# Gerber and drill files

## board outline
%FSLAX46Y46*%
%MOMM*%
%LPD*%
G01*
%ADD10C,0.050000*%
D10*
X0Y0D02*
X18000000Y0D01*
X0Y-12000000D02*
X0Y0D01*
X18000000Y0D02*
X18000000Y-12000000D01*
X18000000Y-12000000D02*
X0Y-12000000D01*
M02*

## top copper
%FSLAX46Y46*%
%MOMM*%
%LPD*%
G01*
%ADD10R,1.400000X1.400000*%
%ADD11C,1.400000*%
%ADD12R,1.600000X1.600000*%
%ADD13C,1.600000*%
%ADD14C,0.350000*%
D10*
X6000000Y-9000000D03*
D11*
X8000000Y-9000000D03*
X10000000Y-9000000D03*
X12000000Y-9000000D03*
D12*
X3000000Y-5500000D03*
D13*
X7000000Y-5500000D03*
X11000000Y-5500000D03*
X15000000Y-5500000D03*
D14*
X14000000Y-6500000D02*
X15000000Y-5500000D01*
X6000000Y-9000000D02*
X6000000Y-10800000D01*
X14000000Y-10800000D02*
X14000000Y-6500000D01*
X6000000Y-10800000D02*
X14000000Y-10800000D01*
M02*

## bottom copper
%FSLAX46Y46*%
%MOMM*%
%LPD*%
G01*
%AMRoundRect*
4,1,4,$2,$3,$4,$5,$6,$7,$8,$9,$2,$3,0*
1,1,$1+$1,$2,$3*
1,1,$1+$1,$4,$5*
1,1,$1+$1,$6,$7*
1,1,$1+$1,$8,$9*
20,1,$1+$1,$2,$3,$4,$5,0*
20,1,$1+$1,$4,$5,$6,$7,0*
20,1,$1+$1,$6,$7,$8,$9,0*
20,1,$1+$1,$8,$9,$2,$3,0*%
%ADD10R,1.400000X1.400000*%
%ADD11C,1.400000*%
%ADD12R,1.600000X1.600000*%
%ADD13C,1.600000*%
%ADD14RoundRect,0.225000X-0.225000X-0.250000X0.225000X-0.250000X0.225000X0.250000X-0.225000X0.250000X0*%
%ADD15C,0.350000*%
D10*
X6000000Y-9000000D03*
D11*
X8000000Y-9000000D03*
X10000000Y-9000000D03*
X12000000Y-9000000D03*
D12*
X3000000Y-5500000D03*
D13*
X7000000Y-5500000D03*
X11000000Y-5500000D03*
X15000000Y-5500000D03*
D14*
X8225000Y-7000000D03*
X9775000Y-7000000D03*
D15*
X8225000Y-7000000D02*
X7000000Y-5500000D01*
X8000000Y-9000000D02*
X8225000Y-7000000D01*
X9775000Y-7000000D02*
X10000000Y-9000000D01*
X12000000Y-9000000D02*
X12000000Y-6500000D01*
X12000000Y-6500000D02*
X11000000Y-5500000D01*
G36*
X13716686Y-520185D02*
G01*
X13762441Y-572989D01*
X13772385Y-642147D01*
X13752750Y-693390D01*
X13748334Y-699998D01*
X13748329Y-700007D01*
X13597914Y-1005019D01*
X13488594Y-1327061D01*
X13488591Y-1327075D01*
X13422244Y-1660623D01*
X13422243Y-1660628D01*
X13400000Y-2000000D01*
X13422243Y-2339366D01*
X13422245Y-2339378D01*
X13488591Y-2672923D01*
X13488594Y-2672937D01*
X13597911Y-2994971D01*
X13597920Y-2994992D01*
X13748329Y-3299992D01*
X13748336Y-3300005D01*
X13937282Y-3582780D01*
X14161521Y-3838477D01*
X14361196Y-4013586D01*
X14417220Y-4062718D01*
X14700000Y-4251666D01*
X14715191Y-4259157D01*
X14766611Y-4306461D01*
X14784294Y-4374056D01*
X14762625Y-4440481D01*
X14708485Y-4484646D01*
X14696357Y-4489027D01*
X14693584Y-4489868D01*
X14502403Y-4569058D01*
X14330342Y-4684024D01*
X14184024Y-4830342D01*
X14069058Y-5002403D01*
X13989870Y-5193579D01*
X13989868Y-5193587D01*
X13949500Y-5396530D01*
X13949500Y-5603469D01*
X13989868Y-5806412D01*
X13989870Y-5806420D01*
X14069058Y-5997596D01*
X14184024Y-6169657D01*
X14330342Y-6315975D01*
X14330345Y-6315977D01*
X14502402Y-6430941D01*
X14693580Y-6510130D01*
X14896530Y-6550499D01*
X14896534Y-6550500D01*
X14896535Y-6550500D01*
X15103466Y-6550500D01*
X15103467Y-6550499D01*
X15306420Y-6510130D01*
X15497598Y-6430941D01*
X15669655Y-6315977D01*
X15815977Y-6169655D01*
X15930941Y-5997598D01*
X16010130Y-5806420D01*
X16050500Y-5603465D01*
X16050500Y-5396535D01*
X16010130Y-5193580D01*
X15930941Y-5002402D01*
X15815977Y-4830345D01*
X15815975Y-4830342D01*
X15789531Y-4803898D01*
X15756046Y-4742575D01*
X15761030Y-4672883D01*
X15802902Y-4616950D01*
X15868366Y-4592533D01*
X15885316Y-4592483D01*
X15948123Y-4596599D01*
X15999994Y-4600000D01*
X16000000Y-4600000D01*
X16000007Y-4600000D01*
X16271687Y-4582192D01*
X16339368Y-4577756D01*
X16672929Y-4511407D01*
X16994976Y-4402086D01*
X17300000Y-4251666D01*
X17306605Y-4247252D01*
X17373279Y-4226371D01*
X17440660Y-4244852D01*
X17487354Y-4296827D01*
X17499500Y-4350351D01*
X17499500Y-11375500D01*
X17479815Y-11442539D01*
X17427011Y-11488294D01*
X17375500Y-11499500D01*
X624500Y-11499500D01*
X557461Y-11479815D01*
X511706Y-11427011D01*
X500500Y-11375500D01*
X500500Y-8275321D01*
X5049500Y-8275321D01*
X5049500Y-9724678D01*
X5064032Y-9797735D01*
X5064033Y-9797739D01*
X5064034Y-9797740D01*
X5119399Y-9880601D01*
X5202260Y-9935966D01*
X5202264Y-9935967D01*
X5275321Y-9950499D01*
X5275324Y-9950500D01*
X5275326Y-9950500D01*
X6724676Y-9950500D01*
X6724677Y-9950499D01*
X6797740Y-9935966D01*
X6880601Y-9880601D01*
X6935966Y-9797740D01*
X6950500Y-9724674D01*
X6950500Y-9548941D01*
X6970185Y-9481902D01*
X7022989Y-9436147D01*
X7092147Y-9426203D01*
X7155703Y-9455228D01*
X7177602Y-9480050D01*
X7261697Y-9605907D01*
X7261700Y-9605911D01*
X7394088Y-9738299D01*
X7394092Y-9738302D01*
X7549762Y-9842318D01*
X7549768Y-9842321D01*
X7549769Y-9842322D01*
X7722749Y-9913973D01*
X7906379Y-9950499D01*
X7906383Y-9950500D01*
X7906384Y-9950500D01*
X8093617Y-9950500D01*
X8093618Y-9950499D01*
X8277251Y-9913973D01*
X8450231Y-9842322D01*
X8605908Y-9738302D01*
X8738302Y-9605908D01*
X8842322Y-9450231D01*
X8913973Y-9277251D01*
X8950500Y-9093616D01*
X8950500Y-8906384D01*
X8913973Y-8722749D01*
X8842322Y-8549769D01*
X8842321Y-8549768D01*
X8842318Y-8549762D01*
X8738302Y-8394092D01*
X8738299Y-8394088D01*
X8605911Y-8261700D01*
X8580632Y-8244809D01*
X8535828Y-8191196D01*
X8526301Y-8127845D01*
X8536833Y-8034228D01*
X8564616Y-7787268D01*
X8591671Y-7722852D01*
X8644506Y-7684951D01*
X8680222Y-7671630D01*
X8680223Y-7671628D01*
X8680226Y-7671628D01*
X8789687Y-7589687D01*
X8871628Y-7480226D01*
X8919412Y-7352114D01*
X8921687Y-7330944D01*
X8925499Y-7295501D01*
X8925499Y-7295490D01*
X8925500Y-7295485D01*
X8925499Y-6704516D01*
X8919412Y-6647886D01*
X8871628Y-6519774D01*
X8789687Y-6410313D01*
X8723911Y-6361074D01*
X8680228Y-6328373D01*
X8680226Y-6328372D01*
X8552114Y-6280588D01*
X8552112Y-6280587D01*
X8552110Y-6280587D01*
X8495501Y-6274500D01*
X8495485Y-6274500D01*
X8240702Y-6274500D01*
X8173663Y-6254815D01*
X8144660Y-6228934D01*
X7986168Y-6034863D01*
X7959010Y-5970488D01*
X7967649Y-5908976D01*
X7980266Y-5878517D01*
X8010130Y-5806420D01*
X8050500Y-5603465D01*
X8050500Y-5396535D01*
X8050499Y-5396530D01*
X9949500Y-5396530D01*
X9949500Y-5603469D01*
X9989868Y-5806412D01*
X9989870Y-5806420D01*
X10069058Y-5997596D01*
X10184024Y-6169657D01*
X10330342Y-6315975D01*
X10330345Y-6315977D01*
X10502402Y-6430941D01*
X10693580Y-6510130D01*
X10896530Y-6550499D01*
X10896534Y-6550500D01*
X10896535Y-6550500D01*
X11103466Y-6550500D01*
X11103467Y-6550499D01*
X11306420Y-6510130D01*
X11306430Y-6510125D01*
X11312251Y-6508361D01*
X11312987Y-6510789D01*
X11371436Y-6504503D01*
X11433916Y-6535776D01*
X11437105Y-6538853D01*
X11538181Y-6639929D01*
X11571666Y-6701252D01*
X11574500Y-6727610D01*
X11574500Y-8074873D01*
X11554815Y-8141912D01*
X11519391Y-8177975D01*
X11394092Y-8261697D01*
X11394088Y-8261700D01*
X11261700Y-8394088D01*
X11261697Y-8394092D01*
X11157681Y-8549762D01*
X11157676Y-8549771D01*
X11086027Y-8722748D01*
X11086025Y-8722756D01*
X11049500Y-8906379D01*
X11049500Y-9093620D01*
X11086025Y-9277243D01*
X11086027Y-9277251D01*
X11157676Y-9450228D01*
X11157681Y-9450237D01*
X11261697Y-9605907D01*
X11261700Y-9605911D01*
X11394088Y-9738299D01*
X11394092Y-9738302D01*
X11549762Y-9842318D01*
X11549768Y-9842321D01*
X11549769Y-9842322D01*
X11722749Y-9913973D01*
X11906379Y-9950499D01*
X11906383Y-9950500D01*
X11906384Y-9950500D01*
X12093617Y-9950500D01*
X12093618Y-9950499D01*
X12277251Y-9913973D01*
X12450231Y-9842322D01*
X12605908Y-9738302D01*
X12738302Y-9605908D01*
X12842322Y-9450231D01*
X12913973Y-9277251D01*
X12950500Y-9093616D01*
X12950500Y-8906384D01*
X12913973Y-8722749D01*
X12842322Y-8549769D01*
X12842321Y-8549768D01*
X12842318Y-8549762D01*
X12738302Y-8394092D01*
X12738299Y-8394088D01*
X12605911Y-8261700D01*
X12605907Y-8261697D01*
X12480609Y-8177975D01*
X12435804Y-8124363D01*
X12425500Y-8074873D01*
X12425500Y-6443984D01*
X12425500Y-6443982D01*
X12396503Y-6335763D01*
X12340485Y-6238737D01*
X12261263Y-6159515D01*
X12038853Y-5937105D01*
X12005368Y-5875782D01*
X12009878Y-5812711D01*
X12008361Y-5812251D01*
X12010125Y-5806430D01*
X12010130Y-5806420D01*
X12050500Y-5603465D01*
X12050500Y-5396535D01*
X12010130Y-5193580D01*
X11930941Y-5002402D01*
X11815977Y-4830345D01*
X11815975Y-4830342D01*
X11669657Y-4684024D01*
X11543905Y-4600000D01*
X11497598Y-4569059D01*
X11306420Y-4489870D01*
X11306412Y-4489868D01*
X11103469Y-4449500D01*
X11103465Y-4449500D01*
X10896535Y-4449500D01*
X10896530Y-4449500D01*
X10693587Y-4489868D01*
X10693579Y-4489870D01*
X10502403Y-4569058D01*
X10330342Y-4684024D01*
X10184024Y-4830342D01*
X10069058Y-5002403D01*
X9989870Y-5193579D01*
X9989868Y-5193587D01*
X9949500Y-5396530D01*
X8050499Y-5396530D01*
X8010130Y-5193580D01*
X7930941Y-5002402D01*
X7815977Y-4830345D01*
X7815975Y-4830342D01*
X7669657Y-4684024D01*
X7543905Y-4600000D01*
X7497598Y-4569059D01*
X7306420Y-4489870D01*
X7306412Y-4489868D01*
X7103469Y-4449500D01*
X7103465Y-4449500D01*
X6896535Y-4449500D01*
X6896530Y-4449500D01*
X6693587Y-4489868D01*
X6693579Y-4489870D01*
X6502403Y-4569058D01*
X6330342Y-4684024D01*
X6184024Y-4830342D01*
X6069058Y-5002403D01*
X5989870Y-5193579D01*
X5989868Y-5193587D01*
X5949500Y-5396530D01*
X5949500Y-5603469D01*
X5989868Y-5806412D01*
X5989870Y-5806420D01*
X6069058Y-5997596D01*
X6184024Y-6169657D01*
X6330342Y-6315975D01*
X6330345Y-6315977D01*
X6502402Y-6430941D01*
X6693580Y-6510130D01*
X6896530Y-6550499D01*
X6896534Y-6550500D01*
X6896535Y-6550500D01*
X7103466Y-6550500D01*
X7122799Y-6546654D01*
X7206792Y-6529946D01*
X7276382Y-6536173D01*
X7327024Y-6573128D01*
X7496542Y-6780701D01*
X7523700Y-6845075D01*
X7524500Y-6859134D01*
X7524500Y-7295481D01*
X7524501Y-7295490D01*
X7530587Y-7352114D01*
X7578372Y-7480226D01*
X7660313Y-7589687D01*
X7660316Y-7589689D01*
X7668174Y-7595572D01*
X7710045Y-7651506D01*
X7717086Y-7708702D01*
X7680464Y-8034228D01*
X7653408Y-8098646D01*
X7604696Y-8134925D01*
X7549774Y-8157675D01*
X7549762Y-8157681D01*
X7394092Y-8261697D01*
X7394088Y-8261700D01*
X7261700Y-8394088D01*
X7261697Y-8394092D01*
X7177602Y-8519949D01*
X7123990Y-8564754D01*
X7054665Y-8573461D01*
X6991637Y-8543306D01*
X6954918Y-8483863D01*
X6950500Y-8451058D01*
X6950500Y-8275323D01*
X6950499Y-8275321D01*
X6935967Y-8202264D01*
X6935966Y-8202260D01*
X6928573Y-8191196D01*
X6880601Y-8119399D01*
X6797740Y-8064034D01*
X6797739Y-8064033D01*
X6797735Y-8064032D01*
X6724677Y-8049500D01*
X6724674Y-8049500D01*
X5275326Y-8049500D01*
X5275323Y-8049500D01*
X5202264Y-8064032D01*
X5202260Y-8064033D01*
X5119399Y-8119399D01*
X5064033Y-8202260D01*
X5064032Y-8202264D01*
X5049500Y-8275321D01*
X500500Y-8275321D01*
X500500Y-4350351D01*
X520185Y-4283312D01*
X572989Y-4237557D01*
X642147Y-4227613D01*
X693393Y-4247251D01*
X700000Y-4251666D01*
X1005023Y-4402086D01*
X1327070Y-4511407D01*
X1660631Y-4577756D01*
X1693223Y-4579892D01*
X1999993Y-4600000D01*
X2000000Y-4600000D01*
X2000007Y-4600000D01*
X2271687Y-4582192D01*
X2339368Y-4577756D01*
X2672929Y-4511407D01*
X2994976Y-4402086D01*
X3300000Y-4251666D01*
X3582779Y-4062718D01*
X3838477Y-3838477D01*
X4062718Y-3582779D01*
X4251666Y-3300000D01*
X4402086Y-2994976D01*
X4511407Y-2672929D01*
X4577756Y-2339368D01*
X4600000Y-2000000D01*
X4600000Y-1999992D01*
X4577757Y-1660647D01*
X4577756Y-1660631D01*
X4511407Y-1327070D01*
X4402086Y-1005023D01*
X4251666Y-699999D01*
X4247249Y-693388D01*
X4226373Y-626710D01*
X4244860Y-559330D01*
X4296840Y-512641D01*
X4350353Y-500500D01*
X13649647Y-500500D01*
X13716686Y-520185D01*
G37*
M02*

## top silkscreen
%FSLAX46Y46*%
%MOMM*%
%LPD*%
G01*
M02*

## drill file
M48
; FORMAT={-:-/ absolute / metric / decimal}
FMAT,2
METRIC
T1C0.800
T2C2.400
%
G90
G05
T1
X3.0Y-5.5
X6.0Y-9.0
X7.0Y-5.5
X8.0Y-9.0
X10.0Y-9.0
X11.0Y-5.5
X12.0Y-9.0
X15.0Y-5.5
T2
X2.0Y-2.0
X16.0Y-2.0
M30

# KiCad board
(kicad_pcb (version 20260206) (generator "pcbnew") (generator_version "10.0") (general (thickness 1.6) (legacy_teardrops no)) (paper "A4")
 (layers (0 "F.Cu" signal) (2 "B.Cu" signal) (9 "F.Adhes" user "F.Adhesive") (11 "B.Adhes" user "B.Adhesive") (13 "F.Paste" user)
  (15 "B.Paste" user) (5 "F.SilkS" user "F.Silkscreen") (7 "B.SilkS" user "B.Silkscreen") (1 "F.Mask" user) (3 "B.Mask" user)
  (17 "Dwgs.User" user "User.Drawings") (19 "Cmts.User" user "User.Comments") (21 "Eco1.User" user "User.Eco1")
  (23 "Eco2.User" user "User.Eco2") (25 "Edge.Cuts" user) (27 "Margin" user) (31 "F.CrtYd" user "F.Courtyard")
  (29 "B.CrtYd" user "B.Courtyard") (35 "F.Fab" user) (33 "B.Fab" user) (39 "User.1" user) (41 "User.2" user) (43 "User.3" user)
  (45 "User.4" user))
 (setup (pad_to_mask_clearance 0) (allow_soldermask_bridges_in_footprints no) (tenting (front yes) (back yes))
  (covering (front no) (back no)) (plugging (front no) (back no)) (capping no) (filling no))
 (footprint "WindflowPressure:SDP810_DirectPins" (layer "F.Cu") (at 9 6)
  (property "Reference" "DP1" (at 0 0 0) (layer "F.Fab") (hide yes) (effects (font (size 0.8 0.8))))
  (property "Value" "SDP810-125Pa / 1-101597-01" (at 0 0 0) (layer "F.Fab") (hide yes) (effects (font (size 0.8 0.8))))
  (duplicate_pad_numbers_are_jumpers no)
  (pad "1" thru_hole rect (at -3 3) (size 1.4 1.4) (drill 0.8) (layers "*.Cu" "*.Mask") (remove_unused_layers no) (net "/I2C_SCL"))
  (pad "2" thru_hole circle (at -1 3) (size 1.4 1.4) (drill 0.8) (layers "*.Cu" "*.Mask") (remove_unused_layers no) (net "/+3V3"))
  (pad "3" thru_hole circle (at 1 3) (size 1.4 1.4) (drill 0.8) (layers "*.Cu" "*.Mask") (remove_unused_layers no) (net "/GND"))
  (pad "4" thru_hole circle (at 3 3) (size 1.4 1.4) (drill 0.8) (layers "*.Cu" "*.Mask") (remove_unused_layers no) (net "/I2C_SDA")))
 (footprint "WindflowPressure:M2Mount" (layer "F.Cu") (at 2 2)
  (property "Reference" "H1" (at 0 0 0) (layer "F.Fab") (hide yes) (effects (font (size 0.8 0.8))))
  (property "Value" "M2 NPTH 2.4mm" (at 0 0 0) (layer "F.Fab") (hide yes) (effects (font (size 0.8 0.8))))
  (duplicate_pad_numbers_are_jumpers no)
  (pad "" np_thru_hole circle (at 0 0) (size 2.4 2.4) (drill 2.4) (layers "*.Cu" "*.Mask")))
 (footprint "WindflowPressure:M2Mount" (layer "F.Cu") (at 16 2)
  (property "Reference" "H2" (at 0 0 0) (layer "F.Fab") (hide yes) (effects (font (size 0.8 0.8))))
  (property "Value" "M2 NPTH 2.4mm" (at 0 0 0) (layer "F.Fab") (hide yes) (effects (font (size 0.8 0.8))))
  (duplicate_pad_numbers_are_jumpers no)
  (pad "" np_thru_hole circle (at 0 0) (size 2.4 2.4) (drill 2.4) (layers "*.Cu" "*.Mask")))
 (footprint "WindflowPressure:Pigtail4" (layer "F.Cu") (at 9 5.5)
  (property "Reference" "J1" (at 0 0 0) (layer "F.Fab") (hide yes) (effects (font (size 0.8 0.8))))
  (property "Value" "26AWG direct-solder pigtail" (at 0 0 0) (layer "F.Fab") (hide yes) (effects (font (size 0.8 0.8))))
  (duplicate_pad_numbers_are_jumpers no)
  (pad "1" thru_hole rect (at -6 0) (size 1.6 1.6) (drill 0.8) (layers "*.Cu" "*.Mask") (remove_unused_layers no) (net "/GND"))
  (pad "2" thru_hole circle (at -2 0) (size 1.6 1.6) (drill 0.8) (layers "*.Cu" "*.Mask") (remove_unused_layers no) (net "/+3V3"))
  (pad "3" thru_hole circle (at 2 0) (size 1.6 1.6) (drill 0.8) (layers "*.Cu" "*.Mask") (remove_unused_layers no) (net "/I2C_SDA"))
  (pad "4" thru_hole circle (at 6 0) (size 1.6 1.6) (drill 0.8) (layers "*.Cu" "*.Mask") (remove_unused_layers no) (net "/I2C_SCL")))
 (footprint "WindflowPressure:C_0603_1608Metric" (layer "B.Cu") (at 9 7)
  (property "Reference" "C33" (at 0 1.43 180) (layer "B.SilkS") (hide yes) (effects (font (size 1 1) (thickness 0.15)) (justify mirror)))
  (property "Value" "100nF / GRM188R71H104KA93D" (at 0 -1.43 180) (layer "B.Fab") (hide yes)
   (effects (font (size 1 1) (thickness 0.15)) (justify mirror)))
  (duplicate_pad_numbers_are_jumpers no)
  (pad "1" smd roundrect (at -0.775 0) (size 0.9 0.95) (layers "B.Cu" "B.Mask" "B.Paste") (roundrect_rratio 0.25) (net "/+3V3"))
  (pad "2" smd roundrect (at 0.775 0) (size 0.9 0.95) (layers "B.Cu" "B.Mask" "B.Paste") (roundrect_rratio 0.25) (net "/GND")))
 (gr_line (start 0 0) (end 18 0) (stroke (width 0.05) (type default)) (layer "Edge.Cuts"))
 (gr_line (start 0 12) (end 0 0) (stroke (width 0.05) (type default)) (layer "Edge.Cuts"))
 (gr_line (start 18 0) (end 18 12) (stroke (width 0.05) (type default)) (layer "Edge.Cuts"))
 (gr_line (start 18 12) (end 0 12) (stroke (width 0.05) (type default)) (layer "Edge.Cuts"))
 (segment (start 14 6.5) (end 15 5.5) (width 0.35) (layer "F.Cu") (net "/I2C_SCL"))
 (segment (start 6 9) (end 6 10.8) (width 0.35) (layer "F.Cu") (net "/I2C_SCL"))
 (segment (start 14 10.8) (end 14 6.5) (width 0.35) (layer "F.Cu") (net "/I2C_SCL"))
 (segment (start 6 10.8) (end 14 10.8) (width 0.35) (layer "F.Cu") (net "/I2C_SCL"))
 (segment (start 8.225 7) (end 7 5.5) (width 0.35) (layer "B.Cu") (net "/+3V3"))
 (segment (start 8 9) (end 8.225 7) (width 0.35) (layer "B.Cu") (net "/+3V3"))
 (segment (start 9.775 7) (end 10 9) (width 0.35) (layer "B.Cu") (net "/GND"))
 (segment (start 12 9) (end 12 6.5) (width 0.35) (layer "B.Cu") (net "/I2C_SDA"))
 (segment (start 12 6.5) (end 11 5.5) (width 0.35) (layer "B.Cu") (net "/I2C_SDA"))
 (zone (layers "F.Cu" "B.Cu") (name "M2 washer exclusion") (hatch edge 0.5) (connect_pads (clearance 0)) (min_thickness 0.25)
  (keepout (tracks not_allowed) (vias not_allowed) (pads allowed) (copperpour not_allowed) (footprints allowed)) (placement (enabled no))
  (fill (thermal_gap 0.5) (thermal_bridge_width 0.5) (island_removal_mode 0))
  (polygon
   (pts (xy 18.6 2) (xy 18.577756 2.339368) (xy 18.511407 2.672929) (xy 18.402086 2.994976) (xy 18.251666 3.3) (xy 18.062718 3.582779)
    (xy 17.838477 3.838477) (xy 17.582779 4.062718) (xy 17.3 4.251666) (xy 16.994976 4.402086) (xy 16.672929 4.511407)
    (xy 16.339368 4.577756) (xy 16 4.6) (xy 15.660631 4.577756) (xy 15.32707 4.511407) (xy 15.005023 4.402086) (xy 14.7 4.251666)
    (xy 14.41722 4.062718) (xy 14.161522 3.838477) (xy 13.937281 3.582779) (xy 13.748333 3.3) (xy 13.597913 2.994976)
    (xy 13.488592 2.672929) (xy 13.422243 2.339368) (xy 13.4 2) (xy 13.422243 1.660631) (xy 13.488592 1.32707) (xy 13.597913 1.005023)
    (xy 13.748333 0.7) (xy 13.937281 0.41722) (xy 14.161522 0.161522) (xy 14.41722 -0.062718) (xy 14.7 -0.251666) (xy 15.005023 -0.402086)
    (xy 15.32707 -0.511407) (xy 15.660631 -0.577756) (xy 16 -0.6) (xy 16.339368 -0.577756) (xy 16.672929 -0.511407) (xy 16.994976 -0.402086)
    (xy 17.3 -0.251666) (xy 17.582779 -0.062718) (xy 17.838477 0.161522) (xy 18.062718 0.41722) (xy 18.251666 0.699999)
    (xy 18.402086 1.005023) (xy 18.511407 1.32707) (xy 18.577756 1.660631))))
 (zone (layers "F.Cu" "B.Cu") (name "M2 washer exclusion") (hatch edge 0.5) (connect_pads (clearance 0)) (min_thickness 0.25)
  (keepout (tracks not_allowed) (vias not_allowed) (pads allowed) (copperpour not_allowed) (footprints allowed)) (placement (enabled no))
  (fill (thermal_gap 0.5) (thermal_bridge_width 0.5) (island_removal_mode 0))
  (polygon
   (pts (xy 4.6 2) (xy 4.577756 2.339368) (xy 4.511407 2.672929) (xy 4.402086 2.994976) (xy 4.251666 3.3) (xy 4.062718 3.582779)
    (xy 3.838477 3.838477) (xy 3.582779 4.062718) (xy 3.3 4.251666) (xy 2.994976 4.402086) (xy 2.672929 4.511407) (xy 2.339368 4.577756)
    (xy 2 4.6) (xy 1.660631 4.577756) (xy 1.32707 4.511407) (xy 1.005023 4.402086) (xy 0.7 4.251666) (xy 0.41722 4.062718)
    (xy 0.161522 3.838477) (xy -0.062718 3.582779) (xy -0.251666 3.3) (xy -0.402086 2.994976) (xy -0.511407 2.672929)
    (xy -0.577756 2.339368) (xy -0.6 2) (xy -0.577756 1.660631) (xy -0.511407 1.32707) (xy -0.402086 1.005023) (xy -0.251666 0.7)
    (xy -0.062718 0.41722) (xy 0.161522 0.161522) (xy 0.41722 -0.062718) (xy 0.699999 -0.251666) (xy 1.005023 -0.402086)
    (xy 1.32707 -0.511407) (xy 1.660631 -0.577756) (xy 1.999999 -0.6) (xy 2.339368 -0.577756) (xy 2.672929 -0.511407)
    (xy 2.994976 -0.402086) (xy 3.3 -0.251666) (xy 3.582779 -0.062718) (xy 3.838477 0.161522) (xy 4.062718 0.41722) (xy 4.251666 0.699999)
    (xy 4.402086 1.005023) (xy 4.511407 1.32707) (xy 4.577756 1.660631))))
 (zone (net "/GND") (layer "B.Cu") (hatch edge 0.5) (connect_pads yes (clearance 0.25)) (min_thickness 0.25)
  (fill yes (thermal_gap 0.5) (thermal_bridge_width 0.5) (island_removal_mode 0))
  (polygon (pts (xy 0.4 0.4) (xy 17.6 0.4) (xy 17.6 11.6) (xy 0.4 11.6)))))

